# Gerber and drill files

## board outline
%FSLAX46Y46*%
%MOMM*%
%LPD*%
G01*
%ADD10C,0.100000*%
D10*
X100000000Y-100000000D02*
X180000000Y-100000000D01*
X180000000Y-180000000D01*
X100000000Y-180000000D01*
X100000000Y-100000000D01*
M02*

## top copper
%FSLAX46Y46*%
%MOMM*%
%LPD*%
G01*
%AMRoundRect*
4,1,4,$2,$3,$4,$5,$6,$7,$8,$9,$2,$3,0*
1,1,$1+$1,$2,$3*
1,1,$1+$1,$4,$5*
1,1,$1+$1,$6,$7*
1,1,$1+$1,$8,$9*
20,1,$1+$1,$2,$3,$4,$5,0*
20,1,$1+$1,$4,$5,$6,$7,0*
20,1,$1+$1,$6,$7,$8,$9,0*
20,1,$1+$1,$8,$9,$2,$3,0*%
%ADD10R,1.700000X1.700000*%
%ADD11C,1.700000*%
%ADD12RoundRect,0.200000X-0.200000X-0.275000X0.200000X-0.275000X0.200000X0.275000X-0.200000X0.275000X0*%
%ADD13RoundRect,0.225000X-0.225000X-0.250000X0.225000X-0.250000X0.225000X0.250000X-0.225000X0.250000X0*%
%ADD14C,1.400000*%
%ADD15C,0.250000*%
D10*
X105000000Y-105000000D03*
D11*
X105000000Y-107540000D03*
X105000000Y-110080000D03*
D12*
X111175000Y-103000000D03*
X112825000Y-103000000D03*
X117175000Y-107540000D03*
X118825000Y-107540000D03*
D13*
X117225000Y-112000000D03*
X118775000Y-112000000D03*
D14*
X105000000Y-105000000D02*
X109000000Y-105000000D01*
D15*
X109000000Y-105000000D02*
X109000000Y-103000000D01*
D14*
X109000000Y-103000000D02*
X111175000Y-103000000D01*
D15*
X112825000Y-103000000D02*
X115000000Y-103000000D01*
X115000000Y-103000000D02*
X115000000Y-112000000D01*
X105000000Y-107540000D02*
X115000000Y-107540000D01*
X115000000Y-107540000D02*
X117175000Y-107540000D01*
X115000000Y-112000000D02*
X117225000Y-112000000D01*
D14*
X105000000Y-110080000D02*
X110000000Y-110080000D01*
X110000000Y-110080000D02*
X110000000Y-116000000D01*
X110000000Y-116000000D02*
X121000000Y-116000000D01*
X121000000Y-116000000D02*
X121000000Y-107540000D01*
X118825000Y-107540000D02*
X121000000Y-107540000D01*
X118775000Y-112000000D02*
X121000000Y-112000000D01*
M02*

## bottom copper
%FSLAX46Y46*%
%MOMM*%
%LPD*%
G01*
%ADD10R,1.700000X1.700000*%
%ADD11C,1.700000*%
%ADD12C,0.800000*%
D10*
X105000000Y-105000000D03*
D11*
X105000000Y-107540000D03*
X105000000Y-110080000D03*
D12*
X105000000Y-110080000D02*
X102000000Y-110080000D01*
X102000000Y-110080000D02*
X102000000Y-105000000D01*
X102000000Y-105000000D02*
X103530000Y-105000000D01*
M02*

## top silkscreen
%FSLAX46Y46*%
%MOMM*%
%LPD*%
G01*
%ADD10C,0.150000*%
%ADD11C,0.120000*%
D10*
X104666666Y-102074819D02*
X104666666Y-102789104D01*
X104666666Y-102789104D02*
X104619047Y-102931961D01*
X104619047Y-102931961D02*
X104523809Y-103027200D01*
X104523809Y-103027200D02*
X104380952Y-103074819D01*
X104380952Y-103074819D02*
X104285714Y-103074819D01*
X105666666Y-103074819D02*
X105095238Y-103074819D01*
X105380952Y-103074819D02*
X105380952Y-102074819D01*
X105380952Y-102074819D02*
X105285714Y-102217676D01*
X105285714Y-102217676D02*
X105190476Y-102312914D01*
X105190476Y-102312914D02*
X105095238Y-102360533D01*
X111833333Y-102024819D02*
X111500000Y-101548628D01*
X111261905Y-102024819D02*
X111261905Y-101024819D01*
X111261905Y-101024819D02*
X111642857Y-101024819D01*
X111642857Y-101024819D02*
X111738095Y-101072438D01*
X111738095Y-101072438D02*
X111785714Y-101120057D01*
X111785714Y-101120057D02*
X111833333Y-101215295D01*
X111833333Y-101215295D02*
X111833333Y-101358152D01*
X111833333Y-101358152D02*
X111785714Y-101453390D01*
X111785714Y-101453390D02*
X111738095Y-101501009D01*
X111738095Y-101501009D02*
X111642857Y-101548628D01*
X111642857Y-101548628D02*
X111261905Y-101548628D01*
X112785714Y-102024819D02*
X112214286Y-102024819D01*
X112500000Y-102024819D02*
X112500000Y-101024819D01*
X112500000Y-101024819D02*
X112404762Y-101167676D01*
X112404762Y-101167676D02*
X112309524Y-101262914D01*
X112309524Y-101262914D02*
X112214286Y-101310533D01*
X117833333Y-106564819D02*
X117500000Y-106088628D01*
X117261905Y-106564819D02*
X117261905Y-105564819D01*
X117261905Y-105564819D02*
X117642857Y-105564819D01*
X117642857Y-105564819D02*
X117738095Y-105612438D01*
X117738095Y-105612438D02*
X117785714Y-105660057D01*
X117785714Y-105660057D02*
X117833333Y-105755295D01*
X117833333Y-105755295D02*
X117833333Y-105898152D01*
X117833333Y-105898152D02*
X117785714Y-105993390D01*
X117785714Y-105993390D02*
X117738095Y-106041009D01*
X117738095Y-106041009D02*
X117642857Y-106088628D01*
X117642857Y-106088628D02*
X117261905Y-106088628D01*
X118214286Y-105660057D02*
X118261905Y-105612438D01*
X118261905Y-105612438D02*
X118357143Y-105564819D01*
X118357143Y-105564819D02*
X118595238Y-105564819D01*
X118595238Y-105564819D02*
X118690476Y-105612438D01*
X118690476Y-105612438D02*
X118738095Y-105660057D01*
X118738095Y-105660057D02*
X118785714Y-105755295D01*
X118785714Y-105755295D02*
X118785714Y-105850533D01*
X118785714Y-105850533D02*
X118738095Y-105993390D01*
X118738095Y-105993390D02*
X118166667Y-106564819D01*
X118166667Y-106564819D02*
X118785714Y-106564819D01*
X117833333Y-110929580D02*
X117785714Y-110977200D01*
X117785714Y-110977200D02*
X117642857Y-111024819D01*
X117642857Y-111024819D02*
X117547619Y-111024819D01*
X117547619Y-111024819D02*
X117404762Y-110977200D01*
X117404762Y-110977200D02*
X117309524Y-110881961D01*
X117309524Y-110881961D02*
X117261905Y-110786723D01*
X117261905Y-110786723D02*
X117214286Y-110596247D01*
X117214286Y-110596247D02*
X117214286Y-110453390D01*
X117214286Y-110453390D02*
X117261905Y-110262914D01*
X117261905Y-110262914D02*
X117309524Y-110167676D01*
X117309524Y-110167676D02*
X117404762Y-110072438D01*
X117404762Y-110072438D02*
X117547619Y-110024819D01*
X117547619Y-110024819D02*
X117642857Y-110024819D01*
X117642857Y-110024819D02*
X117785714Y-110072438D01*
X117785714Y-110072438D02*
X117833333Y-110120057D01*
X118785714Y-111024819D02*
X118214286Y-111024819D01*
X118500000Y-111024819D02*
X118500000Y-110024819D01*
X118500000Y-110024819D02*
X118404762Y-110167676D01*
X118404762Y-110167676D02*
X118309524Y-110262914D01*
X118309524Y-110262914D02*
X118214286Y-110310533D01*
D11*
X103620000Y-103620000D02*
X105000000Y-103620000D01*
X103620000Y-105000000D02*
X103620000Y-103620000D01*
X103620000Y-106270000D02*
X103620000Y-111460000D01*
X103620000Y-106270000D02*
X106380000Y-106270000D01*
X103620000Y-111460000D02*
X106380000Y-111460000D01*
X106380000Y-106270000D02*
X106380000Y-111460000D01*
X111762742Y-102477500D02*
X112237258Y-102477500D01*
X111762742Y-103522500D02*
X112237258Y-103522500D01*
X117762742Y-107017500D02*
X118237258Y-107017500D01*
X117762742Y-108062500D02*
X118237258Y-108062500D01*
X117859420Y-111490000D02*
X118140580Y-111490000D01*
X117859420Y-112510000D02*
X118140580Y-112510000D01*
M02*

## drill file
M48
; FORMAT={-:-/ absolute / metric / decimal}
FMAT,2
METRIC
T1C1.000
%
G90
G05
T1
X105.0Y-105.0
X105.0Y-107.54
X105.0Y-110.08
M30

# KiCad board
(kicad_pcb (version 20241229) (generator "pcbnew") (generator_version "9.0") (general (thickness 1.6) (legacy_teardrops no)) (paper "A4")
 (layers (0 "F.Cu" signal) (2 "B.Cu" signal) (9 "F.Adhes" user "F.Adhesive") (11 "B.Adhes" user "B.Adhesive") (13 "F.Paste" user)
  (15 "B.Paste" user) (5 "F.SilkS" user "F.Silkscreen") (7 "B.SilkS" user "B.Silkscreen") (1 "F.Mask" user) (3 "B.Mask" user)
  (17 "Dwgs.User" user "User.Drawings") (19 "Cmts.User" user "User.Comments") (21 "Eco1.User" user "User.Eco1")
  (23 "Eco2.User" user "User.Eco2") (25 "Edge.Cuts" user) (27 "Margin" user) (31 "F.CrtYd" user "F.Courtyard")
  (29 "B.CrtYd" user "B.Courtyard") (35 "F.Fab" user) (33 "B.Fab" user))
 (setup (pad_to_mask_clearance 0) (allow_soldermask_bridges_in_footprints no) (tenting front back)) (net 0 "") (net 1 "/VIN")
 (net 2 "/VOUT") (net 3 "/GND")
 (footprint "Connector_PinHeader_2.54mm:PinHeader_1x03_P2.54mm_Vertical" (layer "F.Cu") (at 105 105)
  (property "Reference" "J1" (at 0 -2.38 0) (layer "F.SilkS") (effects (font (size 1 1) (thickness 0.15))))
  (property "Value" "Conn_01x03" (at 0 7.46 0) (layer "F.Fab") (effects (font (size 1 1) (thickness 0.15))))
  (fp_line (start -1.38 -1.38) (end 0 -1.38) (stroke (width 0.12) (type solid)) (layer "F.SilkS"))
  (fp_line (start -1.38 0) (end -1.38 -1.38) (stroke (width 0.12) (type solid)) (layer "F.SilkS"))
  (fp_line (start -1.38 1.27) (end -1.38 6.46) (stroke (width 0.12) (type solid)) (layer "F.SilkS"))
  (fp_line (start -1.38 1.27) (end 1.38 1.27) (stroke (width 0.12) (type solid)) (layer "F.SilkS"))
  (fp_line (start -1.38 6.46) (end 1.38 6.46) (stroke (width 0.12) (type solid)) (layer "F.SilkS"))
  (fp_line (start 1.38 1.27) (end 1.38 6.46) (stroke (width 0.12) (type solid)) (layer "F.SilkS"))
  (pad "1" thru_hole rect (at 0 0) (size 1.7 1.7) (drill 1) (layers "*.Cu" "*.Mask") (remove_unused_layers no) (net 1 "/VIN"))
  (pad "2" thru_hole circle (at 0 2.54) (size 1.7 1.7) (drill 1) (layers "*.Cu" "*.Mask") (remove_unused_layers no) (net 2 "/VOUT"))
  (pad "3" thru_hole circle (at 0 5.08) (size 1.7 1.7) (drill 1) (layers "*.Cu" "*.Mask") (remove_unused_layers no) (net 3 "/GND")))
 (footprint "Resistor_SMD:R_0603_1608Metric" (layer "F.Cu") (at 112 103)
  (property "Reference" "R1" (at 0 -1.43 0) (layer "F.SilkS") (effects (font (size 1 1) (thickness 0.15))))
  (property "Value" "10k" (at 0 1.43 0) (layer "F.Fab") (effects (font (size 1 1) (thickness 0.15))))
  (fp_line (start -0.237258 -0.5225) (end 0.237258 -0.5225) (stroke (width 0.12) (type solid)) (layer "F.SilkS"))
  (fp_line (start -0.237258 0.5225) (end 0.237258 0.5225) (stroke (width 0.12) (type solid)) (layer "F.SilkS"))
  (pad "1" smd roundrect (at -0.825 0) (size 0.8 0.95) (layers "F.Cu" "F.Mask" "F.Paste") (roundrect_rratio 0.25) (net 1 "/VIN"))
  (pad "2" smd roundrect (at 0.825 0) (size 0.8 0.95) (layers "F.Cu" "F.Mask" "F.Paste") (roundrect_rratio 0.25) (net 2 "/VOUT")))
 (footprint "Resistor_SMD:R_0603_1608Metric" (layer "F.Cu") (at 118 107.54)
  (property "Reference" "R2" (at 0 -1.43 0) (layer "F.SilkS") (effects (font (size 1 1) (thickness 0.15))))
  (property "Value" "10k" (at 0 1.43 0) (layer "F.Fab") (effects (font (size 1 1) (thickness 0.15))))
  (fp_line (start -0.237258 -0.5225) (end 0.237258 -0.5225) (stroke (width 0.12) (type solid)) (layer "F.SilkS"))
  (fp_line (start -0.237258 0.5225) (end 0.237258 0.5225) (stroke (width 0.12) (type solid)) (layer "F.SilkS"))
  (pad "1" smd roundrect (at -0.825 0) (size 0.8 0.95) (layers "F.Cu" "F.Mask" "F.Paste") (roundrect_rratio 0.25) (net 2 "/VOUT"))
  (pad "2" smd roundrect (at 0.825 0) (size 0.8 0.95) (layers "F.Cu" "F.Mask" "F.Paste") (roundrect_rratio 0.25) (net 3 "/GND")))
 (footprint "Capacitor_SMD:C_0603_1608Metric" (layer "F.Cu") (at 118 112)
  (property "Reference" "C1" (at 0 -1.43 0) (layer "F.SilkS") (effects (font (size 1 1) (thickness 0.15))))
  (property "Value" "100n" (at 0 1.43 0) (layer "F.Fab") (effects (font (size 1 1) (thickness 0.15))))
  (fp_line (start -0.14058 -0.51) (end 0.14058 -0.51) (stroke (width 0.12) (type solid)) (layer "F.SilkS"))
  (fp_line (start -0.14058 0.51) (end 0.14058 0.51) (stroke (width 0.12) (type solid)) (layer "F.SilkS"))
  (pad "1" smd roundrect (at -0.775 0) (size 0.9 0.95) (layers "F.Cu" "F.Mask" "F.Paste") (roundrect_rratio 0.25) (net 2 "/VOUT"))
  (pad "2" smd roundrect (at 0.775 0) (size 0.9 0.95) (layers "F.Cu" "F.Mask" "F.Paste") (roundrect_rratio 0.25) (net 3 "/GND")))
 (gr_rect (start 100 100) (end 180 180) (stroke (width 0.1) (type default)) (fill no) (layer "Edge.Cuts"))
 (segment (start 105 105) (end 109 105) (width 1.4) (layer "F.Cu") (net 1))
 (segment (start 109 105) (end 109 103) (width 0.25) (layer "F.Cu") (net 1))
 (segment (start 109 103) (end 111.175 103) (width 1.4) (layer "F.Cu") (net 1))
 (segment (start 112.825 103) (end 115 103) (width 0.25) (layer "F.Cu") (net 2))
 (segment (start 115 103) (end 115 112) (width 0.25) (layer "F.Cu") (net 2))
 (segment (start 105 107.54) (end 115 107.54) (width 0.25) (layer "F.Cu") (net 2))
 (segment (start 115 107.54) (end 117.175 107.54) (width 0.25) (layer "F.Cu") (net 2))
 (segment (start 115 112) (end 117.225 112) (width 0.25) (layer "F.Cu") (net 2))
 (segment (start 105 110.08) (end 110 110.08) (width 1.4) (layer "F.Cu") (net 3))
 (segment (start 110 110.08) (end 110 116) (width 1.4) (layer "F.Cu") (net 3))
 (segment (start 110 116) (end 121 116) (width 1.4) (layer "F.Cu") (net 3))
 (segment (start 121 116) (end 121 107.54) (width 1.4) (layer "F.Cu") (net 3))
 (segment (start 118.825 107.54) (end 121 107.54) (width 1.4) (layer "F.Cu") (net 3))
 (segment (start 118.775 112) (end 121 112) (width 1.4) (layer "F.Cu") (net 3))
 (segment (start 105 110.08) (end 102 110.08) (width 0.8) (layer "B.Cu") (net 3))
 (segment (start 102 110.08) (end 102 105) (width 0.8) (layer "B.Cu") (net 3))
 (segment (start 102 105) (end 103.53 105) (width 0.8) (layer "B.Cu") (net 3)))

